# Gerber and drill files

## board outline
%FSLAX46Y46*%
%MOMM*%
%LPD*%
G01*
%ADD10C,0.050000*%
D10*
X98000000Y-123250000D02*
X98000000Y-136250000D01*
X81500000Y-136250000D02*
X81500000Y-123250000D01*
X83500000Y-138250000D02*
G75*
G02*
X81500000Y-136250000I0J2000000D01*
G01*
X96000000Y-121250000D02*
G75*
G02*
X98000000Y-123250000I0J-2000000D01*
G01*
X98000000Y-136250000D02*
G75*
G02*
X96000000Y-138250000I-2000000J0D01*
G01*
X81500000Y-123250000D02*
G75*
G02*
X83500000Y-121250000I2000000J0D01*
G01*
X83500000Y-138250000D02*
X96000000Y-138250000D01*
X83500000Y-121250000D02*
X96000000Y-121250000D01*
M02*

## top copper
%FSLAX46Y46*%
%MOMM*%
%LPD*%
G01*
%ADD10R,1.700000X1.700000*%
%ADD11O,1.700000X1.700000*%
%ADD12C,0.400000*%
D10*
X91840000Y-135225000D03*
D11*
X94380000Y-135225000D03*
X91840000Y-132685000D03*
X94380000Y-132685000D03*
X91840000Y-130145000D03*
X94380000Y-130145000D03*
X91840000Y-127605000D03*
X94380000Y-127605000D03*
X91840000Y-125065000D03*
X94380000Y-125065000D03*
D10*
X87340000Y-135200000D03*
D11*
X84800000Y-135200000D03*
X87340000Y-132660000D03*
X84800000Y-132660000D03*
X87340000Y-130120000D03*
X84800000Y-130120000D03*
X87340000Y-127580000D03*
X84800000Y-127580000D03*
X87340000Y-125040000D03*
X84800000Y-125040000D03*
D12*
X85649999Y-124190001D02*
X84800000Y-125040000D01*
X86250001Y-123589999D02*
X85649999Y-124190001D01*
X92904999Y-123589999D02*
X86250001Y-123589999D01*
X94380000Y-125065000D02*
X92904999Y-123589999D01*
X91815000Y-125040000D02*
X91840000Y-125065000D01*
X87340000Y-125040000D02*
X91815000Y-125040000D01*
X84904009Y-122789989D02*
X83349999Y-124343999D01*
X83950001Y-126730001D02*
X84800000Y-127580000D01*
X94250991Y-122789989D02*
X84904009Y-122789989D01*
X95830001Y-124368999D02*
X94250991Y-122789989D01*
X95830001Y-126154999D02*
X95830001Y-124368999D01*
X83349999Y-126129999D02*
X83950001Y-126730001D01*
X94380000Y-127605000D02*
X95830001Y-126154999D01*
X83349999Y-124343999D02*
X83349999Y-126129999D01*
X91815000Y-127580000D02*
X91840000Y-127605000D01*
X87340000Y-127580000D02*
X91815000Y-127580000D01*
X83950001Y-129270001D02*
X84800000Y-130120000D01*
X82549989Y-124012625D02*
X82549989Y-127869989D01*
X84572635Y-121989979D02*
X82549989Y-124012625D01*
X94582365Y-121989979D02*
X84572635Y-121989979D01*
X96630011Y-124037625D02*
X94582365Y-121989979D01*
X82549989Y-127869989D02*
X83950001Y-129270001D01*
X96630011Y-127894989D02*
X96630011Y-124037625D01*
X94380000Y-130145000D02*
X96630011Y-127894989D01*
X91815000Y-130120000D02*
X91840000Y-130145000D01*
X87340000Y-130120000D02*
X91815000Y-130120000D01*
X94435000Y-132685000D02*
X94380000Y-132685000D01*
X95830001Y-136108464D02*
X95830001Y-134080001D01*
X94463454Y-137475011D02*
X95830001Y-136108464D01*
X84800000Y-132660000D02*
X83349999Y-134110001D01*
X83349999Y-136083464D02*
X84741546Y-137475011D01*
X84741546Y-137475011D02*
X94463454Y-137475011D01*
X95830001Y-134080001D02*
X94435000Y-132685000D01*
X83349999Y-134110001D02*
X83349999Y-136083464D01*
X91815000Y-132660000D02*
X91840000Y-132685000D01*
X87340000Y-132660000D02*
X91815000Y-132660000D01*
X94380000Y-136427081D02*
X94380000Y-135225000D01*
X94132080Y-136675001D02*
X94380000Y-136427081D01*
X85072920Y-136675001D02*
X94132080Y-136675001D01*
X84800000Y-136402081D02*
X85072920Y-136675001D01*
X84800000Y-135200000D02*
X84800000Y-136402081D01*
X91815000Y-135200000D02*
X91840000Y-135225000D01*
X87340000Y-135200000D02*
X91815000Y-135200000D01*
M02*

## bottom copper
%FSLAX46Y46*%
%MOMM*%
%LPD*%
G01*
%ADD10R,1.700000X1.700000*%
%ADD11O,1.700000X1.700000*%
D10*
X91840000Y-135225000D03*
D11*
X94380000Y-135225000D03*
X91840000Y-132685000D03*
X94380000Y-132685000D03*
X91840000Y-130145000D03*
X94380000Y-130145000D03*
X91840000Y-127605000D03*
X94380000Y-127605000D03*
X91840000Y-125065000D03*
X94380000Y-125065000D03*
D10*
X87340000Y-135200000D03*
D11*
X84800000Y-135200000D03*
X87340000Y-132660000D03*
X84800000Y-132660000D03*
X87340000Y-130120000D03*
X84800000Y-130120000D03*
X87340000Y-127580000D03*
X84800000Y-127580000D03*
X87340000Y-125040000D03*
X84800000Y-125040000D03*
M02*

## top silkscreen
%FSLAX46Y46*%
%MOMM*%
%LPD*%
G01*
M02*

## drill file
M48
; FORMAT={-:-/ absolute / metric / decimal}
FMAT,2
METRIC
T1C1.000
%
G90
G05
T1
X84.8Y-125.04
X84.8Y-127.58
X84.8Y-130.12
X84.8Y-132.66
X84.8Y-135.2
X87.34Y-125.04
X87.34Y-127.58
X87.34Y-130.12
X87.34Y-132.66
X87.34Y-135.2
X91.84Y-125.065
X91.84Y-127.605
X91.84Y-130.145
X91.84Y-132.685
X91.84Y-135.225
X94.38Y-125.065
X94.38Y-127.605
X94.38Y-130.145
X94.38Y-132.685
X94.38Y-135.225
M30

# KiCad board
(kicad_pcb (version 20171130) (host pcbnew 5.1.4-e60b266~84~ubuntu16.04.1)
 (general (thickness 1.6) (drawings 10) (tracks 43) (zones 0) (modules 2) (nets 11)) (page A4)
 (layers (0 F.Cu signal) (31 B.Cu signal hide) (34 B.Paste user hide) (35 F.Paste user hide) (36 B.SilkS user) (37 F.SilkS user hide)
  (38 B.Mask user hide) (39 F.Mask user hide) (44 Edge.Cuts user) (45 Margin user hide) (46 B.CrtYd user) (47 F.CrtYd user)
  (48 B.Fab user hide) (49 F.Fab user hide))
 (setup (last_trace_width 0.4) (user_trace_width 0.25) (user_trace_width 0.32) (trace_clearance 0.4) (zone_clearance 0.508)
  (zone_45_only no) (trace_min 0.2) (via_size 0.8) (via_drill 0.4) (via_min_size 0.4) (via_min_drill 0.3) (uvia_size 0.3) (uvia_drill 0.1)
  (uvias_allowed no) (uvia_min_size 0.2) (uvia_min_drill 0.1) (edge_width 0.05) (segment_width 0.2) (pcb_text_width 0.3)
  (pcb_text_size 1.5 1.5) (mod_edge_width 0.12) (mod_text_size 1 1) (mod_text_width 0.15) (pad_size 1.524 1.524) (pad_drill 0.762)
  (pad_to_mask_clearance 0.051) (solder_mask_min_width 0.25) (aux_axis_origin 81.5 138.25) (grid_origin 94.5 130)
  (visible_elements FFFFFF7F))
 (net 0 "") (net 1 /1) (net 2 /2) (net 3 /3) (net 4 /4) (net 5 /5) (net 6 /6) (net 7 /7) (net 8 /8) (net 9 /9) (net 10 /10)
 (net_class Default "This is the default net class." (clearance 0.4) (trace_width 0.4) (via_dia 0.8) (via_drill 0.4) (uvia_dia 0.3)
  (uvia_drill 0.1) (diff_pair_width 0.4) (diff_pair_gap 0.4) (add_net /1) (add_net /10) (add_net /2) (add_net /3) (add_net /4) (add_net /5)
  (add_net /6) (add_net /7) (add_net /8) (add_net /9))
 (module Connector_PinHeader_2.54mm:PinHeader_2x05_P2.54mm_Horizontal (layer B.Cu) (at 91.84 135.225)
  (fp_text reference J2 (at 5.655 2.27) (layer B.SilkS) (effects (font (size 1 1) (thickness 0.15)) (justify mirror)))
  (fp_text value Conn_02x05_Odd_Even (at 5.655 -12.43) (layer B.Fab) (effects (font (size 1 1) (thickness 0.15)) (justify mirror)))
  (pad 1 thru_hole rect (at 0 0) (size 1.7 1.7) (drill 1) (layers *.Cu *.Mask) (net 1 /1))
  (pad 2 thru_hole oval (at 2.54 0) (size 1.7 1.7) (drill 1) (layers *.Cu *.Mask) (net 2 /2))
  (pad 3 thru_hole oval (at 0 -2.54) (size 1.7 1.7) (drill 1) (layers *.Cu *.Mask) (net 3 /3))
  (pad 4 thru_hole oval (at 2.54 -2.54) (size 1.7 1.7) (drill 1) (layers *.Cu *.Mask) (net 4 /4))
  (pad 5 thru_hole oval (at 0 -5.08) (size 1.7 1.7) (drill 1) (layers *.Cu *.Mask) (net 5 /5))
  (pad 6 thru_hole oval (at 2.54 -5.08) (size 1.7 1.7) (drill 1) (layers *.Cu *.Mask) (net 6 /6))
  (pad 7 thru_hole oval (at 0 -7.62) (size 1.7 1.7) (drill 1) (layers *.Cu *.Mask) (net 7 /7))
  (pad 8 thru_hole oval (at 2.54 -7.62) (size 1.7 1.7) (drill 1) (layers *.Cu *.Mask) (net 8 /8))
  (pad 9 thru_hole oval (at 0 -10.16) (size 1.7 1.7) (drill 1) (layers *.Cu *.Mask) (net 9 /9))
  (pad 10 thru_hole oval (at 2.54 -10.16) (size 1.7 1.7) (drill 1) (layers *.Cu *.Mask) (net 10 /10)))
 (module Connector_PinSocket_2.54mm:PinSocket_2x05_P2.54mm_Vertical (layer B.Cu) (at 87.34 135.2)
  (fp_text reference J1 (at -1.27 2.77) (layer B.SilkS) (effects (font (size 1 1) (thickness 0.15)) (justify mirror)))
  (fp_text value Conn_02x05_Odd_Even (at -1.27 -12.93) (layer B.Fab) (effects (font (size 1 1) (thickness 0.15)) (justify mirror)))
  (pad 1 thru_hole rect (at 0 0) (size 1.7 1.7) (drill 1) (layers *.Cu *.Mask) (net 1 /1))
  (pad 2 thru_hole oval (at -2.54 0) (size 1.7 1.7) (drill 1) (layers *.Cu *.Mask) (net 2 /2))
  (pad 3 thru_hole oval (at 0 -2.54) (size 1.7 1.7) (drill 1) (layers *.Cu *.Mask) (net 3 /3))
  (pad 4 thru_hole oval (at -2.54 -2.54) (size 1.7 1.7) (drill 1) (layers *.Cu *.Mask) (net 4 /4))
  (pad 5 thru_hole oval (at 0 -5.08) (size 1.7 1.7) (drill 1) (layers *.Cu *.Mask) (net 5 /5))
  (pad 6 thru_hole oval (at -2.54 -5.08) (size 1.7 1.7) (drill 1) (layers *.Cu *.Mask) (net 6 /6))
  (pad 7 thru_hole oval (at 0 -7.62) (size 1.7 1.7) (drill 1) (layers *.Cu *.Mask) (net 7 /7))
  (pad 8 thru_hole oval (at -2.54 -7.62) (size 1.7 1.7) (drill 1) (layers *.Cu *.Mask) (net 8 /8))
  (pad 9 thru_hole oval (at 0 -10.16) (size 1.7 1.7) (drill 1) (layers *.Cu *.Mask) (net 9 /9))
  (pad 10 thru_hole oval (at -2.54 -10.16) (size 1.7 1.7) (drill 1) (layers *.Cu *.Mask) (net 10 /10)))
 (gr_line (start 98 123.25) (end 98 136.25) (layer Edge.Cuts) (width 0.05))
 (gr_line (start 81.5 136.25) (end 81.5 123.25) (layer Edge.Cuts) (width 0.05))
 (gr_arc (start 83.5 136.25) (end 81.5 136.25) (angle -90) (layer Edge.Cuts) (width 0.05))
 (gr_arc (start 96 123.25) (end 98 123.25) (angle -90) (layer Edge.Cuts) (width 0.05))
 (gr_arc (start 96 136.25) (end 96 138.25) (angle -90) (layer Edge.Cuts) (width 0.05))
 (gr_arc (start 83.5 123.25) (end 83.5 121.25) (angle -90) (layer Edge.Cuts) (width 0.05))
 (gr_line (start 83.5 138.25) (end 96 138.25) (layer Edge.Cuts) (width 0.05))
 (gr_line (start 83.5 121.25) (end 96 121.25) (layer Edge.Cuts) (width 0.05))
 (segment (start 85.649999 124.190001) (end 84.8 125.04) (width 0.4) (layer F.Cu) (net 10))
 (segment (start 86.250001 123.589999) (end 85.649999 124.190001) (width 0.4) (layer F.Cu) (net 10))
 (segment (start 92.904999 123.589999) (end 86.250001 123.589999) (width 0.4) (layer F.Cu) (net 10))
 (segment (start 94.38 125.065) (end 92.904999 123.589999) (width 0.4) (layer F.Cu) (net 10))
 (segment (start 91.815 125.04) (end 91.84 125.065) (width 0.4) (layer F.Cu) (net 9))
 (segment (start 87.34 125.04) (end 91.815 125.04) (width 0.4) (layer F.Cu) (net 9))
 (segment (start 84.904009 122.789989) (end 83.349999 124.343999) (width 0.4) (layer F.Cu) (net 8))
 (segment (start 83.950001 126.730001) (end 84.8 127.58) (width 0.4) (layer F.Cu) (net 8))
 (segment (start 94.250991 122.789989) (end 84.904009 122.789989) (width 0.4) (layer F.Cu) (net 8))
 (segment (start 95.830001 124.368999) (end 94.250991 122.789989) (width 0.4) (layer F.Cu) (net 8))
 (segment (start 95.830001 126.154999) (end 95.830001 124.368999) (width 0.4) (layer F.Cu) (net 8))
 (segment (start 83.349999 126.129999) (end 83.950001 126.730001) (width 0.4) (layer F.Cu) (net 8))
 (segment (start 94.38 127.605) (end 95.830001 126.154999) (width 0.4) (layer F.Cu) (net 8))
 (segment (start 83.349999 124.343999) (end 83.349999 126.129999) (width 0.4) (layer F.Cu) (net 8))
 (segment (start 91.815 127.58) (end 91.84 127.605) (width 0.4) (layer F.Cu) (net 7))
 (segment (start 87.34 127.58) (end 91.815 127.58) (width 0.4) (layer F.Cu) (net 7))
 (segment (start 83.950001 129.270001) (end 84.8 130.12) (width 0.4) (layer F.Cu) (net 6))
 (segment (start 82.549989 124.012625) (end 82.549989 127.869989) (width 0.4) (layer F.Cu) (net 6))
 (segment (start 84.572635 121.989979) (end 82.549989 124.012625) (width 0.4) (layer F.Cu) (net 6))
 (segment (start 94.582365 121.989979) (end 84.572635 121.989979) (width 0.4) (layer F.Cu) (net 6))
 (segment (start 96.630011 124.037625) (end 94.582365 121.989979) (width 0.4) (layer F.Cu) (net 6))
 (segment (start 82.549989 127.869989) (end 83.950001 129.270001) (width 0.4) (layer F.Cu) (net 6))
 (segment (start 96.630011 127.894989) (end 96.630011 124.037625) (width 0.4) (layer F.Cu) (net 6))
 (segment (start 94.38 130.145) (end 96.630011 127.894989) (width 0.4) (layer F.Cu) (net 6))
 (segment (start 91.815 130.12) (end 91.84 130.145) (width 0.4) (layer F.Cu) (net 5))
 (segment (start 87.34 130.12) (end 91.815 130.12) (width 0.4) (layer F.Cu) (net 5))
 (segment (start 94.435 132.685) (end 94.38 132.685) (width 0.4) (layer F.Cu) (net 4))
 (segment (start 95.830001 136.108464) (end 95.830001 134.080001) (width 0.4) (layer F.Cu) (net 4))
 (segment (start 94.463454 137.475011) (end 95.830001 136.108464) (width 0.4) (layer F.Cu) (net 4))
 (segment (start 84.8 132.66) (end 83.349999 134.110001) (width 0.4) (layer F.Cu) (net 4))
 (segment (start 83.349999 136.083464) (end 84.741546 137.475011) (width 0.4) (layer F.Cu) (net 4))
 (segment (start 84.741546 137.475011) (end 94.463454 137.475011) (width 0.4) (layer F.Cu) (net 4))
 (segment (start 95.830001 134.080001) (end 94.435 132.685) (width 0.4) (layer F.Cu) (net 4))
 (segment (start 83.349999 134.110001) (end 83.349999 136.083464) (width 0.4) (layer F.Cu) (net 4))
 (segment (start 91.815 132.66) (end 91.84 132.685) (width 0.4) (layer F.Cu) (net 3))
 (segment (start 87.34 132.66) (end 91.815 132.66) (width 0.4) (layer F.Cu) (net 3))
 (segment (start 94.38 136.427081) (end 94.38 135.225) (width 0.4) (layer F.Cu) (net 2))
 (segment (start 94.13208 136.675001) (end 94.38 136.427081) (width 0.4) (layer F.Cu) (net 2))
 (segment (start 85.07292 136.675001) (end 94.13208 136.675001) (width 0.4) (layer F.Cu) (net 2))
 (segment (start 84.8 136.402081) (end 85.07292 136.675001) (width 0.4) (layer F.Cu) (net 2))
 (segment (start 84.8 135.2) (end 84.8 136.402081) (width 0.4) (layer F.Cu) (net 2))
 (segment (start 91.815 135.2) (end 91.84 135.225) (width 0.4) (layer F.Cu) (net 1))
 (segment (start 87.34 135.2) (end 91.815 135.2) (width 0.4) (layer F.Cu) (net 1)))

